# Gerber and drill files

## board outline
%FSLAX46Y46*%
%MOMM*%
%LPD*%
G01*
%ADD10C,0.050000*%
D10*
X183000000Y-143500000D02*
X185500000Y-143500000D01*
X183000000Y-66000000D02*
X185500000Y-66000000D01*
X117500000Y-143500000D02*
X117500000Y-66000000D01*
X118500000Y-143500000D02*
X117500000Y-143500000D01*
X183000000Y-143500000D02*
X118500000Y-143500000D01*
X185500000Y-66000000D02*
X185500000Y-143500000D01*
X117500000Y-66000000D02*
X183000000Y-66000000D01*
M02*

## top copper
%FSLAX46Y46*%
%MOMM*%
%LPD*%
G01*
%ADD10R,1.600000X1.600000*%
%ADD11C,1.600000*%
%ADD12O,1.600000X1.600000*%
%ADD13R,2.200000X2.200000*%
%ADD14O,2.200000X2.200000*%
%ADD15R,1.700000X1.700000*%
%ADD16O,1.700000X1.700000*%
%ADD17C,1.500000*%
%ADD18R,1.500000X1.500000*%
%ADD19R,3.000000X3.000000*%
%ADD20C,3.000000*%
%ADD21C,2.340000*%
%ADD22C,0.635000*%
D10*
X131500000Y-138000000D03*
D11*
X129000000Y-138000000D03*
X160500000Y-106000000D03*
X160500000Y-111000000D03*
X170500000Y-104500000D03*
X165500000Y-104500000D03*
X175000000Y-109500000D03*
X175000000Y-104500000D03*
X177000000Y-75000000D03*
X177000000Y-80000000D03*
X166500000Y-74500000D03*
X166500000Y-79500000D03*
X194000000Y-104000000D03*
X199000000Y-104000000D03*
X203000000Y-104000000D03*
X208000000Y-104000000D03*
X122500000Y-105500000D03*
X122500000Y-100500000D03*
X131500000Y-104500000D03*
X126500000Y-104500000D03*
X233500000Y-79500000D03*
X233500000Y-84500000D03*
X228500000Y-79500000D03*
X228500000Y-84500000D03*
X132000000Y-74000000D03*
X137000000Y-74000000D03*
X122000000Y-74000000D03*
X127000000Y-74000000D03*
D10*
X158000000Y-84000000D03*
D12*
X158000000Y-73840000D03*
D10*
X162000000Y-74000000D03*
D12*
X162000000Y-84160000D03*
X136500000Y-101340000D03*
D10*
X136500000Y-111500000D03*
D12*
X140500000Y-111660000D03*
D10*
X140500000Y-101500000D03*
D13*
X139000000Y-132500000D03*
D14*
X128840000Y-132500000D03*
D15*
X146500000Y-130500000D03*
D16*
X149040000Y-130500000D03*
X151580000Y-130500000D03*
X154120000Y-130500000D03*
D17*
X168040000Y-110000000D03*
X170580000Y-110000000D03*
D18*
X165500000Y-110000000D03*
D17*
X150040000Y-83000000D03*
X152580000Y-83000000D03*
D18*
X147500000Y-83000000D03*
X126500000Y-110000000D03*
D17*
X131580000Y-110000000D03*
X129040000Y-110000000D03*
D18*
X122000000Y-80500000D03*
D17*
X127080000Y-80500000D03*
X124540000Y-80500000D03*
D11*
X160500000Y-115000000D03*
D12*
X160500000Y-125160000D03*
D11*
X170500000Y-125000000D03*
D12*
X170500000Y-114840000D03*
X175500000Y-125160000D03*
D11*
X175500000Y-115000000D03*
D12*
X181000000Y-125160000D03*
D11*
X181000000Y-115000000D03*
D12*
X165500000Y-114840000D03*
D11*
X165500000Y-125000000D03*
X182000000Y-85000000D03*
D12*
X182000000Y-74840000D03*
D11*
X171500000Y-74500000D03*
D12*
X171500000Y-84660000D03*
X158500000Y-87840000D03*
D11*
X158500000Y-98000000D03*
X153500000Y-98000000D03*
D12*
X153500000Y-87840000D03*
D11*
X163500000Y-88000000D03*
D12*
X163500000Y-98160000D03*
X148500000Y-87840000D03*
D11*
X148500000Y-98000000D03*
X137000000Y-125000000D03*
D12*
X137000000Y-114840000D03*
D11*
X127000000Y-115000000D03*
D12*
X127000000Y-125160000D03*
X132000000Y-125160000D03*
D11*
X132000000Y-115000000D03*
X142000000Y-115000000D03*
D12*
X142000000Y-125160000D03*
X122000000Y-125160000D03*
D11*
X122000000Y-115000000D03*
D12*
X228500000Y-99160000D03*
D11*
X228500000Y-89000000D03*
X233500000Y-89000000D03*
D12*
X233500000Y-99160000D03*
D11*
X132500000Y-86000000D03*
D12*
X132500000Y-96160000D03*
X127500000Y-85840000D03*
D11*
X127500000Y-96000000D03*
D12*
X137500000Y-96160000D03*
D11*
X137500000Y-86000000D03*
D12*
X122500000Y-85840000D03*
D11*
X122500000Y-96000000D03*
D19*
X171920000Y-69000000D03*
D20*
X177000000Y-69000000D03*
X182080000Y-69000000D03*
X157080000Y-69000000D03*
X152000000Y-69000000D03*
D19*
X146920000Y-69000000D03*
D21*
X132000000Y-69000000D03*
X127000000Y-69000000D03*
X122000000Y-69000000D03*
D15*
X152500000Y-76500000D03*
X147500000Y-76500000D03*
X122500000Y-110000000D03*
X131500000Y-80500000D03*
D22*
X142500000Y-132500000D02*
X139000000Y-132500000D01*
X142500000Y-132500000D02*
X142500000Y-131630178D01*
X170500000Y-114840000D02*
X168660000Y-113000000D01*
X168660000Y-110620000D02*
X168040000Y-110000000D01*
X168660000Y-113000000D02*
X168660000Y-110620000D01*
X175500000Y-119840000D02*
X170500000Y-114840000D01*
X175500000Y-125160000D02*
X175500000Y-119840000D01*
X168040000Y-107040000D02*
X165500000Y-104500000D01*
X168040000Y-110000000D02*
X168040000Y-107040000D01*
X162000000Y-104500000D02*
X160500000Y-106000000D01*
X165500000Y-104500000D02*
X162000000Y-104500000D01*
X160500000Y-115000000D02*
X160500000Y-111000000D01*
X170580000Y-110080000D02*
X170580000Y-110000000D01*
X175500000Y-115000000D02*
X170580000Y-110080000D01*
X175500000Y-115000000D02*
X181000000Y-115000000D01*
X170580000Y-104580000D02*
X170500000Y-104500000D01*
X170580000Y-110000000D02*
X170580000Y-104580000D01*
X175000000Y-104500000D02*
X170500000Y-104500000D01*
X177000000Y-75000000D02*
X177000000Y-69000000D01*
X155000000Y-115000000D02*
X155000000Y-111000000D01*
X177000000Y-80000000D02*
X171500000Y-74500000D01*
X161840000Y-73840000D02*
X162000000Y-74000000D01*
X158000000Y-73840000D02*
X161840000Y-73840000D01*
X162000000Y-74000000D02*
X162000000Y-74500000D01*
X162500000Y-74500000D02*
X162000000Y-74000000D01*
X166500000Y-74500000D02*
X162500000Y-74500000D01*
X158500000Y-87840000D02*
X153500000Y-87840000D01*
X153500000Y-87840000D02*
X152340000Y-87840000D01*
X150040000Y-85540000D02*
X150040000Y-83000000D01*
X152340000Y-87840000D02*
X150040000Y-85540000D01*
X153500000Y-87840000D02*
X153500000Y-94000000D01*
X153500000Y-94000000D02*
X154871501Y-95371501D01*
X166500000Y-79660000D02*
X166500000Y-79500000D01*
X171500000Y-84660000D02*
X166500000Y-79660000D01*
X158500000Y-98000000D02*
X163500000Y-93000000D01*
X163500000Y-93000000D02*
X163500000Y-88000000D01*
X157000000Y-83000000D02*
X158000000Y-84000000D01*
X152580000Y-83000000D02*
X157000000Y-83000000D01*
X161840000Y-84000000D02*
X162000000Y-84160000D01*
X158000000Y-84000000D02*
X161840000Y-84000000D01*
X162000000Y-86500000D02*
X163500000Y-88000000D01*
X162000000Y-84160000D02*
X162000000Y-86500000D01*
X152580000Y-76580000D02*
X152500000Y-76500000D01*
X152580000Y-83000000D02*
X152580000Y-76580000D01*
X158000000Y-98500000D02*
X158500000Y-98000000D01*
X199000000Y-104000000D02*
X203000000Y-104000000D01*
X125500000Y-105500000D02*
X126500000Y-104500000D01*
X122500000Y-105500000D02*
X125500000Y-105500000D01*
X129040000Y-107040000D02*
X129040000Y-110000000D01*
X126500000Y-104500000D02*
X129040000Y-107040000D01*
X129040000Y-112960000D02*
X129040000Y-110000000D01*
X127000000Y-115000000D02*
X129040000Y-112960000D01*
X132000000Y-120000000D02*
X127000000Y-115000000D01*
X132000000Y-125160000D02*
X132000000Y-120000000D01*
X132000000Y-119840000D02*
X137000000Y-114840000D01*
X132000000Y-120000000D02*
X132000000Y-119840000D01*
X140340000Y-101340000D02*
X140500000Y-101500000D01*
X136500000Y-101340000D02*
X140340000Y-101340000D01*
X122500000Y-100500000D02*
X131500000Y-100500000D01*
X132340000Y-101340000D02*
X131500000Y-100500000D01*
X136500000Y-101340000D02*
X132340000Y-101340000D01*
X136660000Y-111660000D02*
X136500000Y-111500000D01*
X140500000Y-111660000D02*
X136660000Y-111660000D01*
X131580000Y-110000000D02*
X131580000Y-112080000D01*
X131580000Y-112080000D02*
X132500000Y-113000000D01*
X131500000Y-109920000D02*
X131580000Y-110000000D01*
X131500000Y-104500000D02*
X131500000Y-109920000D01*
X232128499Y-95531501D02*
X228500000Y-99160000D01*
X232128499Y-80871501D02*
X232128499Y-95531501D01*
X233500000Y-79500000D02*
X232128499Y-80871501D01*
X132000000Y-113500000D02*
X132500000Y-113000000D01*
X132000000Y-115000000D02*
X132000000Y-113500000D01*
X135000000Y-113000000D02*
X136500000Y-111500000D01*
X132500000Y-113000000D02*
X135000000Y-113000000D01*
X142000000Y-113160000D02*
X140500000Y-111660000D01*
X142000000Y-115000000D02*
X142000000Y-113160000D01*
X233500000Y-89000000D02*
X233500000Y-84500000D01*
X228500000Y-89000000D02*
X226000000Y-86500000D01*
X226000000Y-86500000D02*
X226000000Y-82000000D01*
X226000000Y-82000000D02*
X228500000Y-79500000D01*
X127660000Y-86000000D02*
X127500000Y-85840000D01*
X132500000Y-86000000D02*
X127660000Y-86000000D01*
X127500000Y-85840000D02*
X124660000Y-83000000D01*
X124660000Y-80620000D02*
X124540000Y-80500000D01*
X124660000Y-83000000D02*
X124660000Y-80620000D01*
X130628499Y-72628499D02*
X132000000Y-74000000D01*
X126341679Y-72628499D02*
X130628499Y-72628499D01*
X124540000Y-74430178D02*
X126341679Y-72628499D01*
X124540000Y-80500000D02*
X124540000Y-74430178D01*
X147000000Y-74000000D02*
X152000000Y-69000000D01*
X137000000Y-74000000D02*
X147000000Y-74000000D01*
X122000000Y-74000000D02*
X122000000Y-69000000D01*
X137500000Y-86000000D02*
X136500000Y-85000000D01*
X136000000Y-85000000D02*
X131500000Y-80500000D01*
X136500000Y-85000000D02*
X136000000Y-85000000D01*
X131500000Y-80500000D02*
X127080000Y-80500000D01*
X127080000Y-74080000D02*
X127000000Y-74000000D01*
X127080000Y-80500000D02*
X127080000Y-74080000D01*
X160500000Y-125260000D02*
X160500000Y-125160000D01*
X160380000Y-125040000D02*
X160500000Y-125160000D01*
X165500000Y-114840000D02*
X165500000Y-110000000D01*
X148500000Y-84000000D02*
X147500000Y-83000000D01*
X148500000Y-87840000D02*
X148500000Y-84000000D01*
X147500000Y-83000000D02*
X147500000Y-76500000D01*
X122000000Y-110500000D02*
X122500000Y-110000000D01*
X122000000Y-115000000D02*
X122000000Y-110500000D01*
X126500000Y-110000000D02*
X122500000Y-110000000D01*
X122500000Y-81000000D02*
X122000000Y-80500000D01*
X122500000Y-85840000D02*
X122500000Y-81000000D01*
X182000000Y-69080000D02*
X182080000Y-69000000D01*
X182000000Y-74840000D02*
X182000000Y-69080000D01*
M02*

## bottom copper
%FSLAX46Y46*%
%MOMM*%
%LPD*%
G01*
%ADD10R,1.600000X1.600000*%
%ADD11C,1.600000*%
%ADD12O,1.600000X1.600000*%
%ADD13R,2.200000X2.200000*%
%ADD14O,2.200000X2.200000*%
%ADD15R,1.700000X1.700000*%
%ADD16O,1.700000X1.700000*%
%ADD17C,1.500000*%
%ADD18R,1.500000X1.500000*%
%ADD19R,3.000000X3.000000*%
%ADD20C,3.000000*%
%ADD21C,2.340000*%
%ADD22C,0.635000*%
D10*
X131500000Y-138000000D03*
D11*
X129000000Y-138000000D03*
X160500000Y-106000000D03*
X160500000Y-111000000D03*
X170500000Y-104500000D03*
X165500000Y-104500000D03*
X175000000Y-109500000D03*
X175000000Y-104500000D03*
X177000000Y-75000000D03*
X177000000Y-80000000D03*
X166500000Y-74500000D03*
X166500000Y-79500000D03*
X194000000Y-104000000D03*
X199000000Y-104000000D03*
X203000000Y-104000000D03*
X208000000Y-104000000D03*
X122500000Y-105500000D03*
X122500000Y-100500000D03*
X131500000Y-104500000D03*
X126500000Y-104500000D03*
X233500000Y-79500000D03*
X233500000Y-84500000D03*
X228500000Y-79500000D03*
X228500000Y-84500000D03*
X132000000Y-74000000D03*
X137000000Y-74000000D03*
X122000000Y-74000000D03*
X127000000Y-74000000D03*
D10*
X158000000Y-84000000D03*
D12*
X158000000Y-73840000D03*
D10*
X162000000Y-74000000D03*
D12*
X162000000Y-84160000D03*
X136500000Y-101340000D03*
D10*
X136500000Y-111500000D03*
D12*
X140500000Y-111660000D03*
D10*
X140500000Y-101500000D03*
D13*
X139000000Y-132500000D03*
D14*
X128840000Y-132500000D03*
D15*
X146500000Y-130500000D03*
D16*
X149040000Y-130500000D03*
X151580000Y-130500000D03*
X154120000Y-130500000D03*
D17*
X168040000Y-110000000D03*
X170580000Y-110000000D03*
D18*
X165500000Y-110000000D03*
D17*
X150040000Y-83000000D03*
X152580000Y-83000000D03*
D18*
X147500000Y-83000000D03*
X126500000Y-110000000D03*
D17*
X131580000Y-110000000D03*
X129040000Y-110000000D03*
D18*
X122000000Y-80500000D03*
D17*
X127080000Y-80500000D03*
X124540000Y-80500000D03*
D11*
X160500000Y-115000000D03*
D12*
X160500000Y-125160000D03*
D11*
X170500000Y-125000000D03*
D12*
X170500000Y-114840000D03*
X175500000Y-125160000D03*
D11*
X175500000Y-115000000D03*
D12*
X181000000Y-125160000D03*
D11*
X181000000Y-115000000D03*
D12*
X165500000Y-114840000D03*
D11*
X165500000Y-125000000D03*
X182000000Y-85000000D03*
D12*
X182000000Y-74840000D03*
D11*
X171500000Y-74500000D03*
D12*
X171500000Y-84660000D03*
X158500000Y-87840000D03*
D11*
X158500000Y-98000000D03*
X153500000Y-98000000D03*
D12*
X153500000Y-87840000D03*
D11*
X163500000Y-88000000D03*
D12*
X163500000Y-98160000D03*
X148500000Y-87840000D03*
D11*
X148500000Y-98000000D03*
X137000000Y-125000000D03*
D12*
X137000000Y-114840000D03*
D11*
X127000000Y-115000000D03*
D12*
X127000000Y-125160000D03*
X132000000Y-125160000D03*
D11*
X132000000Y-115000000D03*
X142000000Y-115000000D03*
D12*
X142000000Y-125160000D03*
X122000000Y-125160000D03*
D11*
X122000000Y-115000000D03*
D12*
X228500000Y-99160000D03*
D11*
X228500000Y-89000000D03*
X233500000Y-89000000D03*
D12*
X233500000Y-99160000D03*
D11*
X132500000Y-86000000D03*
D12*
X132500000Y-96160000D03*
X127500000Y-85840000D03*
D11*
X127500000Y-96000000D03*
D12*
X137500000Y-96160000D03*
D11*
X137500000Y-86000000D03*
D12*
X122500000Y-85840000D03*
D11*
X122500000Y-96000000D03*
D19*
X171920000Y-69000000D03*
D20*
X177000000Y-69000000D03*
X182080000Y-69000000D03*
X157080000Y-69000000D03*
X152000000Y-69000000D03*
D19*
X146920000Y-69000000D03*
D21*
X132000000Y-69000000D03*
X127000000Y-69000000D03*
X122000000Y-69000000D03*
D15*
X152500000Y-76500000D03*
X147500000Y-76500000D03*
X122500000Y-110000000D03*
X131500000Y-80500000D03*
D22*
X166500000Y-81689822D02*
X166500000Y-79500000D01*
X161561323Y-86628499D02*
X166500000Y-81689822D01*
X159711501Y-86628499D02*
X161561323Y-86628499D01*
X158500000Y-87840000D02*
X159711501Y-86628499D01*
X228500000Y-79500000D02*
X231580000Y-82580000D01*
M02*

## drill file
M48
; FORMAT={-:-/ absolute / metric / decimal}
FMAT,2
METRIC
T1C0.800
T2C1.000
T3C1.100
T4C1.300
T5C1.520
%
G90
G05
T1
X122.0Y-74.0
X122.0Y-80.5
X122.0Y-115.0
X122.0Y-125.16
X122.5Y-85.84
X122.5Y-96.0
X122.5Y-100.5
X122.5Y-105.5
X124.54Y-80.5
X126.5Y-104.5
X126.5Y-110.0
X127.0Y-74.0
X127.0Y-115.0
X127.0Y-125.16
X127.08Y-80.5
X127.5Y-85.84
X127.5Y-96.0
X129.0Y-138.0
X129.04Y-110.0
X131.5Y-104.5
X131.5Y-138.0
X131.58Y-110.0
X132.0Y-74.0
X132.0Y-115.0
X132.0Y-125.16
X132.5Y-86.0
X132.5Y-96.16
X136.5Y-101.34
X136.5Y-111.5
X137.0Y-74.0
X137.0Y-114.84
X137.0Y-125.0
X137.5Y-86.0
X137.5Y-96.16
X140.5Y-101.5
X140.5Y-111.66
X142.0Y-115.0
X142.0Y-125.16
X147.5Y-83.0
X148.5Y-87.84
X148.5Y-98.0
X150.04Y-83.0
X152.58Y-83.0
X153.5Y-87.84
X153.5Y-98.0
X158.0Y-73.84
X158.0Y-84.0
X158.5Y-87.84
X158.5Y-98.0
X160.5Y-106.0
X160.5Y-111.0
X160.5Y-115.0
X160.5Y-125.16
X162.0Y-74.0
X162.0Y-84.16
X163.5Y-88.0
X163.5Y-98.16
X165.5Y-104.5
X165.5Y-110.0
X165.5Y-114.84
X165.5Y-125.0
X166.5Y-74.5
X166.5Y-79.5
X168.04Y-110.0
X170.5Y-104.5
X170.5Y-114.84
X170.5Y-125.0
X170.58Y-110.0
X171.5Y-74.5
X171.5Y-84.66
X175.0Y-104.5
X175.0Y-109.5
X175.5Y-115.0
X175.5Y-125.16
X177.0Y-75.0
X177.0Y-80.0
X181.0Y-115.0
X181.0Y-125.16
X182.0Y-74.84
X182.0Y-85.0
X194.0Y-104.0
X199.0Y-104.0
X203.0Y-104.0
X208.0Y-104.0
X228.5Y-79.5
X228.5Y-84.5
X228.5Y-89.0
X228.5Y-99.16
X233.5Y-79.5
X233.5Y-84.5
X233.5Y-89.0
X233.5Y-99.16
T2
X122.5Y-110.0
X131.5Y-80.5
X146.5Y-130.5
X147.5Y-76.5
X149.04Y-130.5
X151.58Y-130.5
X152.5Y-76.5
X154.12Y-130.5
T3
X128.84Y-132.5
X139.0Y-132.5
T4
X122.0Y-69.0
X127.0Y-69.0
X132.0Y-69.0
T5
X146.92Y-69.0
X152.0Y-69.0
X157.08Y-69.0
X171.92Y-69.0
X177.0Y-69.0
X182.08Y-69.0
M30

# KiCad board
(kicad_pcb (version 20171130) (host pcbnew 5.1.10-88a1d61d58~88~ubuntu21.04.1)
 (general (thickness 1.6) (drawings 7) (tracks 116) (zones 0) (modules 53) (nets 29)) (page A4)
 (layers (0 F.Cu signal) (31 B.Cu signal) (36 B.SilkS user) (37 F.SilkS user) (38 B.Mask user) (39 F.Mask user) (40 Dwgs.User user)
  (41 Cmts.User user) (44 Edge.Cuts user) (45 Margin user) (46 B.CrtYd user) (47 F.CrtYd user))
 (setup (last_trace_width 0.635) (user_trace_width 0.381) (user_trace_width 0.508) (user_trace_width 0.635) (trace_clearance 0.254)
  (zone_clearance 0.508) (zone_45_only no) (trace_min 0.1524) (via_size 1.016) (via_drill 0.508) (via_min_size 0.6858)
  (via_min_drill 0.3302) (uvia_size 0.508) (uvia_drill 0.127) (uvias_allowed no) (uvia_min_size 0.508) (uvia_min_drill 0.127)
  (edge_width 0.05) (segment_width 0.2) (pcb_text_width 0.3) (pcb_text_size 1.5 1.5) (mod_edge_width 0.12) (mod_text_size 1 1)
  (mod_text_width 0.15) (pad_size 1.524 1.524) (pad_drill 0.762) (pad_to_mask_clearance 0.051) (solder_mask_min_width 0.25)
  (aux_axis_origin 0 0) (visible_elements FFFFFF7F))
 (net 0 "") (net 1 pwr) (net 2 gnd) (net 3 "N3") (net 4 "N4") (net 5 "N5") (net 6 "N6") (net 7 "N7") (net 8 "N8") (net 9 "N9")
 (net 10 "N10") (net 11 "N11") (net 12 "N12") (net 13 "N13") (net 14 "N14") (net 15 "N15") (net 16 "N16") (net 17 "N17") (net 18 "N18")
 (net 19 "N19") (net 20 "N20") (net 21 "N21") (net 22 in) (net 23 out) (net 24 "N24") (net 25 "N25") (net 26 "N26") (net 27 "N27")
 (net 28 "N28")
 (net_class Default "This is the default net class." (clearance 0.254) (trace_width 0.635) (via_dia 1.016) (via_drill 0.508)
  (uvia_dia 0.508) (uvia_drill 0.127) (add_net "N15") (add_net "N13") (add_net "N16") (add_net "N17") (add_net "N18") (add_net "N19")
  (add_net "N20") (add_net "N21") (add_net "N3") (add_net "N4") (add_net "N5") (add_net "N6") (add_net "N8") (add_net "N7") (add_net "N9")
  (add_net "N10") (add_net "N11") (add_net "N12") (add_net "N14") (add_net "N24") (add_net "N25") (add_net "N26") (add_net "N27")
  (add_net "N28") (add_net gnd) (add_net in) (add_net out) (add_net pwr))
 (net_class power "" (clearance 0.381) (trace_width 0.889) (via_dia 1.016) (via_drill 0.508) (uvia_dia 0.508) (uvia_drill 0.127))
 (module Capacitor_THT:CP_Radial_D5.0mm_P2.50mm (layer F.Cu) (at 131.5 138 180)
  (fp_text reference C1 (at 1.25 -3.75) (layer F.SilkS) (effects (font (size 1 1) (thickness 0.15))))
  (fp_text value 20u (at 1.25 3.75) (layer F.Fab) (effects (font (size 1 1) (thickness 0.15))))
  (pad 1 thru_hole rect (at 0 0 180) (size 1.6 1.6) (drill 0.8) (layers *.Cu *.Mask) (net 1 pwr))
  (pad 2 thru_hole circle (at 2.5 0 180) (size 1.6 1.6) (drill 0.8) (layers *.Cu *.Mask) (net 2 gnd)))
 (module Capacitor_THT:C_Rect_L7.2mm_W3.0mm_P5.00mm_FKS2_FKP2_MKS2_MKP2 (layer F.Cu) (at 160.5 106 270)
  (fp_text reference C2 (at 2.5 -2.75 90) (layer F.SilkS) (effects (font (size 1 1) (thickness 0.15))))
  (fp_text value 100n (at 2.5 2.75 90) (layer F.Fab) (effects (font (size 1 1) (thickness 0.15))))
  (pad 1 thru_hole circle (at 0 0 270) (size 1.6 1.6) (drill 0.8) (layers *.Cu *.Mask) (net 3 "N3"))
  (pad 2 thru_hole circle (at 5 0 270) (size 1.6 1.6) (drill 0.8) (layers *.Cu *.Mask) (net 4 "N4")))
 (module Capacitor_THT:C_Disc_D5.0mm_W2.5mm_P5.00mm (layer F.Cu) (at 170.5 104.5 180)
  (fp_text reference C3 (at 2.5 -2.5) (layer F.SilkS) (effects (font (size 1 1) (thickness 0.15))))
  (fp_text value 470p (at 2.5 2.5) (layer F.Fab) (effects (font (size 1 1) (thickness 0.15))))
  (pad 1 thru_hole circle (at 0 0 180) (size 1.6 1.6) (drill 0.8) (layers *.Cu *.Mask) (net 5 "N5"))
  (pad 2 thru_hole circle (at 5 0 180) (size 1.6 1.6) (drill 0.8) (layers *.Cu *.Mask) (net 3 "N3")))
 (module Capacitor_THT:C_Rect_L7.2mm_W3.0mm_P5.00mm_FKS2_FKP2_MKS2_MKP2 (layer F.Cu) (at 175 109.5 90)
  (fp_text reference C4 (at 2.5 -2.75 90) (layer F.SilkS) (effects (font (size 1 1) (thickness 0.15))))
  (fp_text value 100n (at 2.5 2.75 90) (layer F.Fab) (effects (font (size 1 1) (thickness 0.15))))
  (pad 1 thru_hole circle (at 0 0 90) (size 1.6 1.6) (drill 0.8) (layers *.Cu *.Mask) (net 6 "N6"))
  (pad 2 thru_hole circle (at 5 0 90) (size 1.6 1.6) (drill 0.8) (layers *.Cu *.Mask) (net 5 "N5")))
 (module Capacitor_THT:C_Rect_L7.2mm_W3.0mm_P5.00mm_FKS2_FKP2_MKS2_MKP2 (layer F.Cu) (at 177 80 90)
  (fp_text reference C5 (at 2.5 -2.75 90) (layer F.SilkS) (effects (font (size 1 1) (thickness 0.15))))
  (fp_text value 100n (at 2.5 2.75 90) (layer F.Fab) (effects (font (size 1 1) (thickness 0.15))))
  (pad 2 thru_hole circle (at 5 0 90) (size 1.6 1.6) (drill 0.8) (layers *.Cu *.Mask) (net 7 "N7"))
  (pad 1 thru_hole circle (at 0 0 90) (size 1.6 1.6) (drill 0.8) (layers *.Cu *.Mask) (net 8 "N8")))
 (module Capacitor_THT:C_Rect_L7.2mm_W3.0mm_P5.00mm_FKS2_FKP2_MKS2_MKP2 (layer F.Cu) (at 166.5 74.5 270)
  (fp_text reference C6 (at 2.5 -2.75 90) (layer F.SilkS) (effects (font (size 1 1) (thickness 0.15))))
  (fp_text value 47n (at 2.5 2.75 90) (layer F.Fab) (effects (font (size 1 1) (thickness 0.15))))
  (pad 1 thru_hole circle (at 0 0 270) (size 1.6 1.6) (drill 0.8) (layers *.Cu *.Mask) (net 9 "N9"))
  (pad 2 thru_hole circle (at 5 0 270) (size 1.6 1.6) (drill 0.8) (layers *.Cu *.Mask) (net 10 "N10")))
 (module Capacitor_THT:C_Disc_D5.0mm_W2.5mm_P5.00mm (layer F.Cu) (at 199 104 180)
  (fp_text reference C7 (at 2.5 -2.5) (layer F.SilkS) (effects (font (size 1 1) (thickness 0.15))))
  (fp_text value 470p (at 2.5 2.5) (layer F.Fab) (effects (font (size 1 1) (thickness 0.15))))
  (pad 2 thru_hole circle (at 5 0 180) (size 1.6 1.6) (drill 0.8) (layers *.Cu *.Mask) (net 10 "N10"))
  (pad 1 thru_hole circle (at 0 0 180) (size 1.6 1.6) (drill 0.8) (layers *.Cu *.Mask) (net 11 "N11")))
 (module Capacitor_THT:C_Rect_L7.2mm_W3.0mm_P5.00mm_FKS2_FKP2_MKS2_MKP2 (layer F.Cu) (at 208 104 180)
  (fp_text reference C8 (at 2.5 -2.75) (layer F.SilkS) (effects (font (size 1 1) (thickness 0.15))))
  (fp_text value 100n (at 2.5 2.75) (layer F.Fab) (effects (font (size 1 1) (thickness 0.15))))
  (pad 2 thru_hole circle (at 5 0 180) (size 1.6 1.6) (drill 0.8) (layers *.Cu *.Mask) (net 11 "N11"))
  (pad 1 thru_hole circle (at 0 0 180) (size 1.6 1.6) (drill 0.8) (layers *.Cu *.Mask) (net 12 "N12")))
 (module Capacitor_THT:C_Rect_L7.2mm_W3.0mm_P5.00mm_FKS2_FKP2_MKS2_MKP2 (layer F.Cu) (at 122.5 100.5 270)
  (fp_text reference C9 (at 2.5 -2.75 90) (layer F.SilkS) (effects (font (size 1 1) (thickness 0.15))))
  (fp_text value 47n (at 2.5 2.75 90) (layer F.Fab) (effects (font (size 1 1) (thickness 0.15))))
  (pad 2 thru_hole circle (at 5 0 270) (size 1.6 1.6) (drill 0.8) (layers *.Cu *.Mask) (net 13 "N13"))
  (pad 1 thru_hole circle (at 0 0 270) (size 1.6 1.6) (drill 0.8) (layers *.Cu *.Mask) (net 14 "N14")))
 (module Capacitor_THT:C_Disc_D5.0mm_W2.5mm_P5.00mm (layer F.Cu) (at 131.5 104.5 180)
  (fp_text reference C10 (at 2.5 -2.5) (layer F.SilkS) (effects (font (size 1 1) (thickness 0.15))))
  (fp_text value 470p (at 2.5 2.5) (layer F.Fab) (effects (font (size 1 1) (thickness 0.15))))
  (pad 1 thru_hole circle (at 0 0 180) (size 1.6 1.6) (drill 0.8) (layers *.Cu *.Mask) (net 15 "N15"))
  (pad 2 thru_hole circle (at 5 0 180) (size 1.6 1.6) (drill 0.8) (layers *.Cu *.Mask) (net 13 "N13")))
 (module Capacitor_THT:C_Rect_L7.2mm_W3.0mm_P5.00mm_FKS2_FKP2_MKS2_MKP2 (layer F.Cu) (at 233.5 84.5 90)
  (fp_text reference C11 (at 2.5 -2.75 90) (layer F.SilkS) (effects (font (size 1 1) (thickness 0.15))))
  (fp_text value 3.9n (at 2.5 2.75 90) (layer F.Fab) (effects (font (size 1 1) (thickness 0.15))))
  (pad 2 thru_hole circle (at 5 0 90) (size 1.6 1.6) (drill 0.8) (layers *.Cu *.Mask) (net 15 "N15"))
  (pad 1 thru_hole circle (at 0 0 90) (size 1.6 1.6) (drill 0.8) (layers *.Cu *.Mask) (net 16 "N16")))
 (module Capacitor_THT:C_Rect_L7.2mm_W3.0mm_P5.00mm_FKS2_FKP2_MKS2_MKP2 (layer F.Cu) (at 228.5 84.5 90)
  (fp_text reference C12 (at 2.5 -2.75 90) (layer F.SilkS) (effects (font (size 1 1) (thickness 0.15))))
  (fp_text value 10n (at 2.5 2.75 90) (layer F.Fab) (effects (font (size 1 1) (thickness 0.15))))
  (pad 2 thru_hole circle (at 5 0 90) (size 1.6 1.6) (drill 0.8) (layers *.Cu *.Mask) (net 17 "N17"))
  (pad 1 thru_hole circle (at 0 0 90) (size 1.6 1.6) (drill 0.8) (layers *.Cu *.Mask) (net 2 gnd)))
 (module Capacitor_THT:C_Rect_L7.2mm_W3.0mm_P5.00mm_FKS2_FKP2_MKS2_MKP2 (layer F.Cu) (at 132 74)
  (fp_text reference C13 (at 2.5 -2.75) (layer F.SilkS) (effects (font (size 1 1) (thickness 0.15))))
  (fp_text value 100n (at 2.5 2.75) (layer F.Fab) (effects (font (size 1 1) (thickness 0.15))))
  (pad 1 thru_hole circle (at 0 0) (size 1.6 1.6) (drill 0.8) (layers *.Cu *.Mask) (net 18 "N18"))
  (pad 2 thru_hole circle (at 5 0) (size 1.6 1.6) (drill 0.8) (layers *.Cu *.Mask) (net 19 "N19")))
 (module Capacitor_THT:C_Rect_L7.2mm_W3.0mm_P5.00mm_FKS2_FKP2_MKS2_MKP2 (layer F.Cu) (at 122 74)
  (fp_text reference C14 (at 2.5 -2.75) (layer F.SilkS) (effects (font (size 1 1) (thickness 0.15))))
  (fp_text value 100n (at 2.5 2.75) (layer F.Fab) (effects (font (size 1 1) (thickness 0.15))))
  (pad 1 thru_hole circle (at 0 0) (size 1.6 1.6) (drill 0.8) (layers *.Cu *.Mask) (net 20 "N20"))
  (pad 2 thru_hole circle (at 5 0) (size 1.6 1.6) (drill 0.8) (layers *.Cu *.Mask) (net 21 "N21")))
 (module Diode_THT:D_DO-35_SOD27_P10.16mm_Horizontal (layer F.Cu) (at 158 84 90)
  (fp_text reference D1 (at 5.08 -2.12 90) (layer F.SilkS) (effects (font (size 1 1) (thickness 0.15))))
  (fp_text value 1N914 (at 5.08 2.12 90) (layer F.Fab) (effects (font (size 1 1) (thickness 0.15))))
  (pad 1 thru_hole rect (at 0 0 90) (size 1.6 1.6) (drill 0.8) (layers *.Cu *.Mask) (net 11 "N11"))
  (pad 2 thru_hole oval (at 10.16 0 90) (size 1.6 1.6) (drill 0.8) (layers *.Cu *.Mask) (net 9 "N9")))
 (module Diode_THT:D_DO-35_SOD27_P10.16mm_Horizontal (layer F.Cu) (at 162 74 270)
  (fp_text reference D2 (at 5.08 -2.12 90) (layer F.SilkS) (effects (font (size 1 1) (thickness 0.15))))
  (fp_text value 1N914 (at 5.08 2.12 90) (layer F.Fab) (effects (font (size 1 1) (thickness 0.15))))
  (pad 1 thru_hole rect (at 0 0 270) (size 1.6 1.6) (drill 0.8) (layers *.Cu *.Mask) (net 9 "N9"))
  (pad 2 thru_hole oval (at 10.16 0 270) (size 1.6 1.6) (drill 0.8) (layers *.Cu *.Mask) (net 11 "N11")))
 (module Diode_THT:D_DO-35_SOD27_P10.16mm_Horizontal (layer F.Cu) (at 136.5 111.5 90)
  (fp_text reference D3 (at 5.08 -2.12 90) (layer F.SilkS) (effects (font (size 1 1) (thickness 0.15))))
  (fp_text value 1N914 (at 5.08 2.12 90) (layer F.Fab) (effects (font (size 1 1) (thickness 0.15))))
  (pad 2 thru_hole oval (at 10.16 0 90) (size 1.6 1.6) (drill 0.8) (layers *.Cu *.Mask) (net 14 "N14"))
  (pad 1 thru_hole rect (at 0 0 90) (size 1.6 1.6) (drill 0.8) (layers *.Cu *.Mask) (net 15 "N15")))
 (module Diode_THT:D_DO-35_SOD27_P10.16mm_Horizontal (layer F.Cu) (at 140.5 101.5 270)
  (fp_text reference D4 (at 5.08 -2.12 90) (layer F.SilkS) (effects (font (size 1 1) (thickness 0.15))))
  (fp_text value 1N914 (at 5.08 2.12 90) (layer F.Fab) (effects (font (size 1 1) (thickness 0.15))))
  (pad 2 thru_hole oval (at 10.16 0 270) (size 1.6 1.6) (drill 0.8) (layers *.Cu *.Mask) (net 15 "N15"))
  (pad 1 thru_hole rect (at 0 0 270) (size 1.6 1.6) (drill 0.8) (layers *.Cu *.Mask) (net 14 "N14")))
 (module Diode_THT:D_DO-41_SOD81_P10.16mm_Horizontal (layer F.Cu) (at 139 132.5 180)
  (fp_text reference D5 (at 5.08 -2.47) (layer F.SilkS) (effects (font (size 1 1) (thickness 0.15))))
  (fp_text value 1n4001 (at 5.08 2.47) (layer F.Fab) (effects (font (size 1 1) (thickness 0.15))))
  (pad 1 thru_hole rect (at 0 0 180) (size 2.2 2.2) (drill 1.1) (layers *.Cu *.Mask) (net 1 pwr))
  (pad 2 thru_hole oval (at 10.16 0 180) (size 2.2 2.2) (drill 1.1) (layers *.Cu *.Mask) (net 2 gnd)))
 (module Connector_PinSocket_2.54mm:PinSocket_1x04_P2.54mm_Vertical (layer F.Cu) (at 146.5 130.5 90)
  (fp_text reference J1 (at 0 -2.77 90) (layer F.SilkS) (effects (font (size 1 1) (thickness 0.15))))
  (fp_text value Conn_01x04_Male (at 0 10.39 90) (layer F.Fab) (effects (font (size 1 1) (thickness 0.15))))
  (pad 1 thru_hole rect (at 0 0 90) (size 1.7 1.7) (drill 1) (layers *.Cu *.Mask) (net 1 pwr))
  (pad 2 thru_hole oval (at 0 2.54 90) (size 1.7 1.7) (drill 1) (layers *.Cu *.Mask) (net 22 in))
  (pad 3 thru_hole oval (at 0 5.08 90) (size 1.7 1.7) (drill 1) (layers *.Cu *.Mask) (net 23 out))
  (pad 4 thru_hole oval (at 0 7.62 90) (size 1.7 1.7) (drill 1) (layers *.Cu *.Mask) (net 2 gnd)))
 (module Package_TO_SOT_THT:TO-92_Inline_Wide (layer F.Cu) (at 165.5 110)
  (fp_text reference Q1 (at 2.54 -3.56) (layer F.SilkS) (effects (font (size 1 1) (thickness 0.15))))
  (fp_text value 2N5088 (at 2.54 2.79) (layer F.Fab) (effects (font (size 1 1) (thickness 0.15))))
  (pad 2 thru_hole circle (at 2.54 0) (size 1.5 1.5) (drill 0.8) (layers *.Cu *.Mask) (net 3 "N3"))
  (pad 3 thru_hole circle (at 5.08 0) (size 1.5 1.5) (drill 0.8) (layers *.Cu *.Mask) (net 5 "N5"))
  (pad 1 thru_hole rect (at 0 0) (size 1.5 1.5) (drill 0.8) (layers *.Cu *.Mask) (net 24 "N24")))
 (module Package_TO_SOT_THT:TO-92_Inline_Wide (layer F.Cu) (at 147.5 83)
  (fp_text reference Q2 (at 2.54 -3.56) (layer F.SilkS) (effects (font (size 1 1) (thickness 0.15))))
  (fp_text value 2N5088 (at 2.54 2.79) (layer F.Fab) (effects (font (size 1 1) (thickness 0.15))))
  (pad 2 thru_hole circle (at 2.54 0) (size 1.5 1.5) (drill 0.8) (layers *.Cu *.Mask) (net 10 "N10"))
  (pad 3 thru_hole circle (at 5.08 0) (size 1.5 1.5) (drill 0.8) (layers *.Cu *.Mask) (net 11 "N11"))
  (pad 1 thru_hole rect (at 0 0) (size 1.5 1.5) (drill 0.8) (layers *.Cu *.Mask) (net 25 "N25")))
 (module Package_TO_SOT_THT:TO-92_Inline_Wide (layer F.Cu) (at 126.5 110)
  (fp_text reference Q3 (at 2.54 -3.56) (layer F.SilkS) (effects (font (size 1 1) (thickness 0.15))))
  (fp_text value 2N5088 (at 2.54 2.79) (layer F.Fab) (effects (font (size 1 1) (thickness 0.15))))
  (pad 1 thru_hole rect (at 0 0) (size 1.5 1.5) (drill 0.8) (layers *.Cu *.Mask) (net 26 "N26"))
  (pad 3 thru_hole circle (at 5.08 0) (size 1.5 1.5) (drill 0.8) (layers *.Cu *.Mask) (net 15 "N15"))
  (pad 2 thru_hole circle (at 2.54 0) (size 1.5 1.5) (drill 0.8) (layers *.Cu *.Mask) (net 13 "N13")))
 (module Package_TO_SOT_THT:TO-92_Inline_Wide (layer F.Cu) (at 122 80.5)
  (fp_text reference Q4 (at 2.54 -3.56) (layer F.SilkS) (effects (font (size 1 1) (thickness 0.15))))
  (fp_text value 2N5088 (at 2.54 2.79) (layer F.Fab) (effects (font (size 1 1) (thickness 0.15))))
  (pad 1 thru_hole rect (at 0 0) (size 1.5 1.5) (drill 0.8) (layers *.Cu *.Mask) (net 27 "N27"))
  (pad 3 thru_hole circle (at 5.08 0) (size 1.5 1.5) (drill 0.8) (layers *.Cu *.Mask) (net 21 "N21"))
  (pad 2 thru_hole circle (at 2.54 0) (size 1.5 1.5) (drill 0.8) (layers *.Cu *.Mask) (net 18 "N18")))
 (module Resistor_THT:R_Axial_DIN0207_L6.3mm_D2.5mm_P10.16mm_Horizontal (layer F.Cu) (at 160.5 115 270)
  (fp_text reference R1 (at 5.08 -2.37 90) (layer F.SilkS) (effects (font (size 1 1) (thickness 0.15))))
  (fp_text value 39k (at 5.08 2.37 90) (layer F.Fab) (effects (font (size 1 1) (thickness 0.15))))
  (pad 1 thru_hole circle (at 0 0 270) (size 1.6 1.6) (drill 0.8) (layers *.Cu *.Mask) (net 4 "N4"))
  (pad 2 thru_hole oval (at 10.16 0 270) (size 1.6 1.6) (drill 0.8) (layers *.Cu *.Mask) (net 22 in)))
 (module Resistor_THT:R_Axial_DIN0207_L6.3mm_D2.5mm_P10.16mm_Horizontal (layer F.Cu) (at 170.5 125 90)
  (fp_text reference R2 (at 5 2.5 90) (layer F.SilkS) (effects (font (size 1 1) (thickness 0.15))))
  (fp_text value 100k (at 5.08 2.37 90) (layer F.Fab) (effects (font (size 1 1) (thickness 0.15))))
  (pad 1 thru_hole circle (at 0 0 90) (size 1.6 1.6) (drill 0.8) (layers *.Cu *.Mask) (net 2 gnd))
  (pad 2 thru_hole oval (at 10.16 0 90) (size 1.6 1.6) (drill 0.8) (layers *.Cu *.Mask) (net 3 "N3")))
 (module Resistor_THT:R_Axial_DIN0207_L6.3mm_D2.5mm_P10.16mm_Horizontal (layer F.Cu) (at 175.5 115 270)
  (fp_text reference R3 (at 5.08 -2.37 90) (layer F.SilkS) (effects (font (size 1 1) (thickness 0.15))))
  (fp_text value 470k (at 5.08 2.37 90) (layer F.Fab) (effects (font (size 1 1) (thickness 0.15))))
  (pad 2 thru_hole oval (at 10.16 0 270) (size 1.6 1.6) (drill 0.8) (layers *.Cu *.Mask) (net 3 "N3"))
  (pad 1 thru_hole circle (at 0 0 270) (size 1.6 1.6) (drill 0.8) (layers *.Cu *.Mask) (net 5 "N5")))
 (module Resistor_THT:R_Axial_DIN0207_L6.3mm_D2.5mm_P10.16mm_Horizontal (layer F.Cu) (at 181 115 270)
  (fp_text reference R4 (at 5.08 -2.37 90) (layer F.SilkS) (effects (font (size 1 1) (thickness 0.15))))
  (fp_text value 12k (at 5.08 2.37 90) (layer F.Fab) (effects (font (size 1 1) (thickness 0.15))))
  (pad 2 thru_hole oval (at 10.16 0 270) (size 1.6 1.6) (drill 0.8) (layers *.Cu *.Mask) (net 1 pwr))
  (pad 1 thru_hole circle (at 0 0 270) (size 1.6 1.6) (drill 0.8) (layers *.Cu *.Mask) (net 5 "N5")))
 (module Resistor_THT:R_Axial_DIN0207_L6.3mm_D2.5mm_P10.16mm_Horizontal (layer F.Cu) (at 165.5 125 90)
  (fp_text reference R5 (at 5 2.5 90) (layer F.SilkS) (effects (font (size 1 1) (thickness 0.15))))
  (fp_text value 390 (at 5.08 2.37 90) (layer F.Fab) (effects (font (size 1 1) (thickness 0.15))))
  (pad 2 thru_hole oval (at 10.16 0 90) (size 1.6 1.6) (drill 0.8) (layers *.Cu *.Mask) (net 24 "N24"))
  (pad 1 thru_hole circle (at 0 0 90) (size 1.6 1.6) (drill 0.8) (layers *.Cu *.Mask) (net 2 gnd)))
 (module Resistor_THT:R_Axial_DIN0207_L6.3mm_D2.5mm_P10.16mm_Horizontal (layer F.Cu) (at 182 85 90)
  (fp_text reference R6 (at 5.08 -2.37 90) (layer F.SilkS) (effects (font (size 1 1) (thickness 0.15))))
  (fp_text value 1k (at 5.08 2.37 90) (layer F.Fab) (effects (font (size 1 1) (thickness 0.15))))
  (pad 1 thru_hole circle (at 0 0 90) (size 1.6 1.6) (drill 0.8) (layers *.Cu *.Mask) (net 2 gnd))
  (pad 2 thru_hole oval (at 10.16 0 90) (size 1.6 1.6) (drill 0.8) (layers *.Cu *.Mask) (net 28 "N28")))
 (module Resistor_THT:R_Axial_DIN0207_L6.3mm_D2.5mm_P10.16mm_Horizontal (layer F.Cu) (at 171.5 74.5 270)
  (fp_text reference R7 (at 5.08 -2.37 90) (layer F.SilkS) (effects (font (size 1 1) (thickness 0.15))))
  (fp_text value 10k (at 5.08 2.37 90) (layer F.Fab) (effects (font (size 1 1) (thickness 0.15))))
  (pad 1 thru_hole circle (at 0 0 270) (size 1.6 1.6) (drill 0.8) (layers *.Cu *.Mask) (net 8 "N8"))
  (pad 2 thru_hole oval (at 10.16 0 270) (size 1.6 1.6) (drill 0.8) (layers *.Cu *.Mask) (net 10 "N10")))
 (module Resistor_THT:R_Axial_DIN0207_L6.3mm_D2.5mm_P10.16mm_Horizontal (layer F.Cu) (at 158.5 98 90)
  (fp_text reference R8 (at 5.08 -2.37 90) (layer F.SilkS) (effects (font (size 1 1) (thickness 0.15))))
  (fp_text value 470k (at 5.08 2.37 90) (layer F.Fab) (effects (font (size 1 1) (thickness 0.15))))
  (pad 2 thru_hole oval (at 10.16 0 90) (size 1.6 1.6) (drill 0.8) (layers *.Cu *.Mask) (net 10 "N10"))
  (pad 1 thru_hole circle (at 0 0 90) (size 1.6 1.6) (drill 0.8) (layers *.Cu *.Mask) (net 11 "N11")))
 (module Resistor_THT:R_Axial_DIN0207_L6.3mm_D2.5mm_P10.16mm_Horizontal (layer F.Cu) (at 153.5 98 90)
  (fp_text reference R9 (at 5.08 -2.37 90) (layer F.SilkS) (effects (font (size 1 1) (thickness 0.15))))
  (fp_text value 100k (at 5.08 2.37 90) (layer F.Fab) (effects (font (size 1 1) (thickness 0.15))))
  (pad 1 thru_hole circle (at 0 0 90) (size 1.6 1.6) (drill 0.8) (layers *.Cu *.Mask) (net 2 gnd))
  (pad 2 thru_hole oval (at 10.16 0 90) (size 1.6 1.6) (drill 0.8) (layers *.Cu *.Mask) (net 10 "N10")))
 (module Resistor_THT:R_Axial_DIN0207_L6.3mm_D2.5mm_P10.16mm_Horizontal (layer F.Cu) (at 163.5 88 270)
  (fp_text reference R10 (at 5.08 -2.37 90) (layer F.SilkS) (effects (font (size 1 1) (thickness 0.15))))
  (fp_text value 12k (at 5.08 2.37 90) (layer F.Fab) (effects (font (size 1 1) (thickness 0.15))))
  (pad 1 thru_hole circle (at 0 0 270) (size 1.6 1.6) (drill 0.8) (layers *.Cu *.Mask) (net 11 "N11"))
  (pad 2 thru_hole oval (at 10.16 0 270) (size 1.6 1.6) (drill 0.8) (layers *.Cu *.Mask) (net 1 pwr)))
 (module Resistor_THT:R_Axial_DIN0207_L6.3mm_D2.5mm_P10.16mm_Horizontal (layer F.Cu) (at 148.5 98 90)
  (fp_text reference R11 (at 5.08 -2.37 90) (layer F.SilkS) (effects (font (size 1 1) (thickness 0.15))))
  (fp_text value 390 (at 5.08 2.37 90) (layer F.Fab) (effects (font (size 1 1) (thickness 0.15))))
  (pad 2 thru_hole oval (at 10.16 0 90) (size 1.6 1.6) (drill 0.8) (layers *.Cu *.Mask) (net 25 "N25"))
  (pad 1 thru_hole circle (at 0 0 90) (size 1.6 1.6) (drill 0.8) (layers *.Cu *.Mask) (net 2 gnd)))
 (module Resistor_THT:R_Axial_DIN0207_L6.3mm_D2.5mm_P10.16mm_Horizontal (layer F.Cu) (at 137 125 90)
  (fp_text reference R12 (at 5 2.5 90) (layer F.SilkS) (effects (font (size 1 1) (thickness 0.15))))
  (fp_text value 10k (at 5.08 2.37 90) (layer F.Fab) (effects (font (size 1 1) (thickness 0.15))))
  (pad 1 thru_hole circle (at 0 0 90) (size 1.6 1.6) (drill 0.8) (layers *.Cu *.Mask) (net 12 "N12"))
  (pad 2 thru_hole oval (at 10.16 0 90) (size 1.6 1.6) (drill 0.8) (layers *.Cu *.Mask) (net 13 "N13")))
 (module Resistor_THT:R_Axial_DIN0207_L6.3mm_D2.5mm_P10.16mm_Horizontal (layer F.Cu) (at 127 115 270)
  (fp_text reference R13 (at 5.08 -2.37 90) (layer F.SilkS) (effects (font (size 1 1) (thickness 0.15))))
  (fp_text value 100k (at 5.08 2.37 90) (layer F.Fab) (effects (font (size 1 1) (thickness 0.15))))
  (pad 1 thru_hole circle (at 0 0 270) (size 1.6 1.6) (drill 0.8) (layers *.Cu *.Mask) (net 13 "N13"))
  (pad 2 thru_hole oval (at 10.16 0 270) (size 1.6 1.6) (drill 0.8) (layers *.Cu *.Mask) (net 2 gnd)))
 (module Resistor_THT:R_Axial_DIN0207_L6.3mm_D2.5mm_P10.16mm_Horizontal (layer F.Cu) (at 132 115 270)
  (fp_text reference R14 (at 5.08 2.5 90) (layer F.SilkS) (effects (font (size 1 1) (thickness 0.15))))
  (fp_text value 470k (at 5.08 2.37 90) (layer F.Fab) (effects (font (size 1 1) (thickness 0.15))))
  (pad 2 thru_hole oval (at 10.16 0 270) (size 1.6 1.6) (drill 0.8) (layers *.Cu *.Mask) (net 13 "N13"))
  (pad 1 thru_hole circle (at 0 0 270) (size 1.6 1.6) (drill 0.8) (layers *.Cu *.Mask) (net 15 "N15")))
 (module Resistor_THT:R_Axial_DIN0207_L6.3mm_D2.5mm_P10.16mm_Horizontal (layer F.Cu) (at 142 115 270)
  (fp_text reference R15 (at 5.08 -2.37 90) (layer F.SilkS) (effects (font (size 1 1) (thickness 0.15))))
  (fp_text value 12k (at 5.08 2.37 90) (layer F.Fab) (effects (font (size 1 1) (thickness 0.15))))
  (pad 1 thru_hole circle (at 0 0 270) (size 1.6 1.6) (drill 0.8) (layers *.Cu *.Mask) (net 15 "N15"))
  (pad 2 thru_hole oval (at 10.16 0 270) (size 1.6 1.6) (drill 0.8) (layers *.Cu *.Mask) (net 1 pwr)))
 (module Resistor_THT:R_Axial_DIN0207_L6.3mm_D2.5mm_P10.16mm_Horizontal (layer F.Cu) (at 122 115 270)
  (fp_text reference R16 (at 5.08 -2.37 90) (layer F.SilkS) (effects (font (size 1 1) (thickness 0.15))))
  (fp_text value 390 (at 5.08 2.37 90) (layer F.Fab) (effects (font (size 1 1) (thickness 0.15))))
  (pad 2 thru_hole oval (at 10.16 0 270) (size 1.6 1.6) (drill 0.8) (layers *.Cu *.Mask) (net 2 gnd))
  (pad 1 thru_hole circle (at 0 0 270) (size 1.6 1.6) (drill 0.8) (layers *.Cu *.Mask) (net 26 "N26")))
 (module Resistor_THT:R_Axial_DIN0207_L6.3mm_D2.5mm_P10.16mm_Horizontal (layer F.Cu) (at 228.5 89 270)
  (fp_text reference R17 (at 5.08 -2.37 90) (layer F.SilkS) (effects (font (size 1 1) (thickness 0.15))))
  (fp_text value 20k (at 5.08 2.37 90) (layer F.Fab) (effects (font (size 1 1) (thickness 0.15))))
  (pad 2 thru_hole oval (at 10.16 0 270) (size 1.6 1.6) (drill 0.8) (layers *.Cu *.Mask) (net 15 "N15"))
  (pad 1 thru_hole circle (at 0 0 270) (size 1.6 1.6) (drill 0.8) (layers *.Cu *.Mask) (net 17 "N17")))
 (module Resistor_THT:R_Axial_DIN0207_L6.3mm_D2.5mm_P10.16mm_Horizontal (layer F.Cu) (at 233.5 89 270)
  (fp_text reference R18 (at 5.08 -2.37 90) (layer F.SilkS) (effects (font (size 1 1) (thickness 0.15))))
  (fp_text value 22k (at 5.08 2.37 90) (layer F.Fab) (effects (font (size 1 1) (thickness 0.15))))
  (pad 1 thru_hole circle (at 0 0 270) (size 1.6 1.6) (drill 0.8) (layers *.Cu *.Mask) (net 16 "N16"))
  (pad 2 thru_hole oval (at 10.16 0 270) (size 1.6 1.6) (drill 0.8) (layers *.Cu *.Mask) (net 2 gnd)))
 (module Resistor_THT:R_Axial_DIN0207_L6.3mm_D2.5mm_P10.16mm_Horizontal (layer F.Cu) (at 132.5 86 270)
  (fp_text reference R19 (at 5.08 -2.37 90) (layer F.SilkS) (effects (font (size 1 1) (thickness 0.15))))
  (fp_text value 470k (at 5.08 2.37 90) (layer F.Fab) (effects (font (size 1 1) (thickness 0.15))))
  (pad 1 thru_hole circle (at 0 0 270) (size 1.6 1.6) (drill 0.8) (layers *.Cu *.Mask) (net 18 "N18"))
  (pad 2 thru_hole oval (at 10.16 0 270) (size 1.6 1.6) (drill 0.8) (layers *.Cu *.Mask) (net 1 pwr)))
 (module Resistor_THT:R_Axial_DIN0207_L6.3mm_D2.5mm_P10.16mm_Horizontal (layer F.Cu) (at 127.5 96 90)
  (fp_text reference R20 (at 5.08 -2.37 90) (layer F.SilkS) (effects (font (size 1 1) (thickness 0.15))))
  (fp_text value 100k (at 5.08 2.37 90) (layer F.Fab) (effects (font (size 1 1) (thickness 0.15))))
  (pad 2 thru_hole oval (at 10.16 0 90) (size 1.6 1.6) (drill 0.8) (layers *.Cu *.Mask) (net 18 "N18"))
  (pad 1 thru_hole circle (at 0 0 90) (size 1.6 1.6) (drill 0.8) (layers *.Cu *.Mask) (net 2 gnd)))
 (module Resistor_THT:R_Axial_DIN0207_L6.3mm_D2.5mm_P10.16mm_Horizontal (layer F.Cu) (at 137.5 86 270)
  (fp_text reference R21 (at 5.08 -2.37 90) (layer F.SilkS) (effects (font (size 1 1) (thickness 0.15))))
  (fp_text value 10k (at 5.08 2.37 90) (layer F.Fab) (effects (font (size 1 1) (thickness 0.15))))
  (pad 2 thru_hole oval (at 10.16 0 270) (size 1.6 1.6) (drill 0.8) (layers *.Cu *.Mask) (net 1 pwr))
  (pad 1 thru_hole circle (at 0 0 270) (size 1.6 1.6) (drill 0.8) (layers *.Cu *.Mask) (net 21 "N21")))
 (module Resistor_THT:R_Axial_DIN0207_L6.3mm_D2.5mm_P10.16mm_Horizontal (layer F.Cu) (at 122.5 96 90)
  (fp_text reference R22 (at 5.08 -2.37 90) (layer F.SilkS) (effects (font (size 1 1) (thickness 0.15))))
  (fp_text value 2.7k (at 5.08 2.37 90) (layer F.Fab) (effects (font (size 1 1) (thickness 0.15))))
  (pad 2 thru_hole oval (at 10.16 0 90) (size 1.6 1.6) (drill 0.8) (layers *.Cu *.Mask) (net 27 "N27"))
  (pad 1 thru_hole circle (at 0 0 90) (size 1.6 1.6) (drill 0.8) (layers *.Cu *.Mask) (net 2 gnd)))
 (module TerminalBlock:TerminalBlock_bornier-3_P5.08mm (layer B.Cu) (at 171.92 69)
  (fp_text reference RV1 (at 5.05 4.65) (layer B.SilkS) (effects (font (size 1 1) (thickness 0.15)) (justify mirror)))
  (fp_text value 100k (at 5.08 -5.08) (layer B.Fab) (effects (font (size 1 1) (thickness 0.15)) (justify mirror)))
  (pad 1 thru_hole rect (at 0 0) (size 3 3) (drill 1.52) (layers *.Cu *.Mask) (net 6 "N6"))
  (pad 2 thru_hole circle (at 5.08 0) (size 3 3) (drill 1.52) (layers *.Cu *.Mask) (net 7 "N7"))
  (pad 3 thru_hole circle (at 10.16 0) (size 3 3) (drill 1.52) (layers *.Cu *.Mask) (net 28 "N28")))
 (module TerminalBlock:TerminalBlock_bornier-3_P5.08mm (layer B.Cu) (at 146.92 69)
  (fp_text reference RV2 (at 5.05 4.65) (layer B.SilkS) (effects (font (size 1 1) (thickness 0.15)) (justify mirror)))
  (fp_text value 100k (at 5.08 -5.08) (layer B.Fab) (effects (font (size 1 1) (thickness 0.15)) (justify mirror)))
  (pad 3 thru_hole circle (at 10.16 0) (size 3 3) (drill 1.52) (layers *.Cu *.Mask) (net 17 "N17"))
  (pad 2 thru_hole circle (at 5.08 0) (size 3 3) (drill 1.52) (layers *.Cu *.Mask) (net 19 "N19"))
  (pad 1 thru_hole rect (at 0 0) (size 3 3) (drill 1.52) (layers *.Cu *.Mask) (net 16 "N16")))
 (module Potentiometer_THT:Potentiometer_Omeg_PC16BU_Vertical (layer B.Cu) (at 122 69 90)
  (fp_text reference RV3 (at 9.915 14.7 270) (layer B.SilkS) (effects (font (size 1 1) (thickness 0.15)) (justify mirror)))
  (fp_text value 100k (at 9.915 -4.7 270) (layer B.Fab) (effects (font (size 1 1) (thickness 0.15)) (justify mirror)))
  (pad 3 thru_hole circle (at 0 10 90) (size 2.34 2.34) (drill 1.3) (layers *.Cu *.Mask) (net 2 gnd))
  (pad 2 thru_hole circle (at 0 5 90) (size 2.34 2.34) (drill 1.3) (layers *.Cu *.Mask) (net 23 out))
  (pad 1 thru_hole circle (at 0 0 90) (size 2.34 2.34) (drill 1.3) (layers *.Cu *.Mask) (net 20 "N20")))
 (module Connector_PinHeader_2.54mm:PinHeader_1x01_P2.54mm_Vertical (layer F.Cu) (at 152.5 76.5)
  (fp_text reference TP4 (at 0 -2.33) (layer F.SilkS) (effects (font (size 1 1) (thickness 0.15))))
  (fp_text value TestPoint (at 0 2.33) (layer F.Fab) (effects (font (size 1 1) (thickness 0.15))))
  (pad 1 thru_hole rect (at 0 0) (size 1.7 1.7) (drill 1) (layers *.Cu *.Mask) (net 11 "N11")))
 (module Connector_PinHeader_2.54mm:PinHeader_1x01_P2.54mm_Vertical (layer F.Cu) (at 147.5 76.5 90)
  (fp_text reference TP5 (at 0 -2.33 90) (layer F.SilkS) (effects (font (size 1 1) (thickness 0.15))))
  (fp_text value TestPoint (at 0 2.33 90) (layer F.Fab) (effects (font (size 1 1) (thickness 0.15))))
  (pad 1 thru_hole rect (at 0 0 90) (size 1.7 1.7) (drill 1) (layers *.Cu *.Mask) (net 25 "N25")))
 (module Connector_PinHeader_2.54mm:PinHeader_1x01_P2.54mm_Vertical (layer F.Cu) (at 122.5 110)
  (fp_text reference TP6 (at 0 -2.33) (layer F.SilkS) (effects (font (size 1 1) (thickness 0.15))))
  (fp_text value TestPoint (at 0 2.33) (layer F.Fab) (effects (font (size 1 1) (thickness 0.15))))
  (pad 1 thru_hole rect (at 0 0) (size 1.7 1.7) (drill 1) (layers *.Cu *.Mask) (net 26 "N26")))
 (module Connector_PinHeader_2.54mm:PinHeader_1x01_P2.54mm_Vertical (layer F.Cu) (at 131.5 80.5)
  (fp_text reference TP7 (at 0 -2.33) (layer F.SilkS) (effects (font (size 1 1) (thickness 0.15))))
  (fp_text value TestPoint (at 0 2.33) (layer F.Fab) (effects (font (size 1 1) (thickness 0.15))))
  (pad 1 thru_hole rect (at 0 0) (size 1.7 1.7) (drill 1) (layers *.Cu *.Mask) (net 21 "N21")))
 (gr_line (start 183 143.5) (end 185.5 143.5) (layer Edge.Cuts) (width 0.05))
 (gr_line (start 183 66) (end 185.5 66) (layer Edge.Cuts) (width 0.05))
 (gr_line (start 117.5 143.5) (end 117.5 66) (layer Edge.Cuts) (width 0.05))
 (gr_line (start 118.5 143.5) (end 117.5 143.5) (layer Edge.Cuts) (width 0.05))
 (gr_line (start 183 143.5) (end 118.5 143.5) (layer Edge.Cuts) (width 0.05))
 (gr_line (start 185.5 66) (end 185.5 143.5) (layer Edge.Cuts) (width 0.05))
 (gr_line (start 117.5 66) (end 183 66) (layer Edge.Cuts) (width 0.05))
 (segment (start 142.5 132.5) (end 139 132.5) (width 0.635) (layer F.Cu) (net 1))
 (segment (start 142.5 132.5) (end 142.5 131.630178) (width 0.635) (layer F.Cu) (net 1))
 (segment (start 170.5 114.84) (end 168.66 113) (width 0.635) (layer F.Cu) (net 3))
 (segment (start 168.66 110.62) (end 168.04 110) (width 0.635) (layer F.Cu) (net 3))
 (segment (start 168.66 113) (end 168.66 110.62) (width 0.635) (layer F.Cu) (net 3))
 (segment (start 175.5 119.84) (end 170.5 114.84) (width 0.635) (layer F.Cu) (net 3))
 (segment (start 175.5 125.16) (end 175.5 119.84) (width 0.635) (layer F.Cu) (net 3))
 (segment (start 168.04 107.04) (end 165.5 104.5) (width 0.635) (layer F.Cu) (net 3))
 (segment (start 168.04 110) (end 168.04 107.04) (width 0.635) (layer F.Cu) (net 3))
 (segment (start 162 104.5) (end 160.5 106) (width 0.635) (layer F.Cu) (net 3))
 (segment (start 165.5 104.5) (end 162 104.5) (width 0.635) (layer F.Cu) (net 3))
 (segment (start 160.5 115) (end 160.5 111) (width 0.635) (layer F.Cu) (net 4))
 (segment (start 170.58 110.08) (end 170.58 110) (width 0.635) (layer F.Cu) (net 5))
 (segment (start 175.5 115) (end 170.58 110.08) (width 0.635) (layer F.Cu) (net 5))
 (segment (start 175.5 115) (end 181 115) (width 0.635) (layer F.Cu) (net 5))
 (segment (start 170.58 104.58) (end 170.5 104.5) (width 0.635) (layer F.Cu) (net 5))
 (segment (start 170.58 110) (end 170.58 104.58) (width 0.635) (layer F.Cu) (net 5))
 (segment (start 175 104.5) (end 170.5 104.5) (width 0.635) (layer F.Cu) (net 5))
 (segment (start 177 75) (end 177 69) (width 0.635) (layer F.Cu) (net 7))
 (segment (start 155 115) (end 155 111) (width 0.635) (layer F.Cu) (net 8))
 (segment (start 177 80) (end 171.5 74.5) (width 0.635) (layer F.Cu) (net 8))
 (segment (start 161.84 73.84) (end 162 74) (width 0.635) (layer F.Cu) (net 9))
 (segment (start 158 73.84) (end 161.84 73.84) (width 0.635) (layer F.Cu) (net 9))
 (segment (start 162 74) (end 162 74.5) (width 0.635) (layer F.Cu) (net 9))
 (segment (start 162.5 74.5) (end 162 74) (width 0.635) (layer F.Cu) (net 9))
 (segment (start 166.5 74.5) (end 162.5 74.5) (width 0.635) (layer F.Cu) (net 9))
 (segment (start 158.5 87.84) (end 153.5 87.84) (width 0.635) (layer F.Cu) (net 10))
 (segment (start 153.5 87.84) (end 152.34 87.84) (width 0.635) (layer F.Cu) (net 10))
 (segment (start 150.04 85.54) (end 150.04 83) (width 0.635) (layer F.Cu) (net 10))
 (segment (start 152.34 87.84) (end 150.04 85.54) (width 0.635) (layer F.Cu) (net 10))
 (segment (start 153.5 87.84) (end 153.5 94) (width 0.635) (layer F.Cu) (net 10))
 (segment (start 153.5 94) (end 154.871501 95.371501) (width 0.635) (layer F.Cu) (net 10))
 (segment (start 166.5 81.689822) (end 166.5 79.5) (width 0.635) (layer B.Cu) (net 10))
 (segment (start 161.561323 86.628499) (end 166.5 81.689822) (width 0.635) (layer B.Cu) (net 10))
 (segment (start 159.711501 86.628499) (end 161.561323 86.628499) (width 0.635) (layer B.Cu) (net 10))
 (segment (start 158.5 87.84) (end 159.711501 86.628499) (width 0.635) (layer B.Cu) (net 10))
 (segment (start 166.5 79.66) (end 166.5 79.5) (width 0.635) (layer F.Cu) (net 10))
 (segment (start 171.5 84.66) (end 166.5 79.66) (width 0.635) (layer F.Cu) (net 10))
 (segment (start 158.5 98) (end 163.5 93) (width 0.635) (layer F.Cu) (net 11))
 (segment (start 163.5 93) (end 163.5 88) (width 0.635) (layer F.Cu) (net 11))
 (segment (start 157 83) (end 158 84) (width 0.635) (layer F.Cu) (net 11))
 (segment (start 152.58 83) (end 157 83) (width 0.635) (layer F.Cu) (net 11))
 (segment (start 161.84 84) (end 162 84.16) (width 0.635) (layer F.Cu) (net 11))
 (segment (start 158 84) (end 161.84 84) (width 0.635) (layer F.Cu) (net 11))
 (segment (start 162 86.5) (end 163.5 88) (width 0.635) (layer F.Cu) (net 11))
 (segment (start 162 84.16) (end 162 86.5) (width 0.635) (layer F.Cu) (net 11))
 (segment (start 152.58 76.58) (end 152.5 76.5) (width 0.635) (layer F.Cu) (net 11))
 (segment (start 152.58 83) (end 152.58 76.58) (width 0.635) (layer F.Cu) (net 11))
 (segment (start 158 98.5) (end 158.5 98) (width 0.635) (layer F.Cu) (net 11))
 (segment (start 199 104) (end 203 104) (width 0.635) (layer F.Cu) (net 11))
 (segment (start 125.5 105.5) (end 126.5 104.5) (width 0.635) (layer F.Cu) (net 13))
 (segment (start 122.5 105.5) (end 125.5 105.5) (width 0.635) (layer F.Cu) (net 13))
 (segment (start 129.04 107.04) (end 129.04 110) (width 0.635) (layer F.Cu) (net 13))
 (segment (start 126.5 104.5) (end 129.04 107.04) (width 0.635) (layer F.Cu) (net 13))
 (segment (start 129.04 112.96) (end 129.04 110) (width 0.635) (layer F.Cu) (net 13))
 (segment (start 127 115) (end 129.04 112.96) (width 0.635) (layer F.Cu) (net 13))
 (segment (start 132 120) (end 127 115) (width 0.635) (layer F.Cu) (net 13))
 (segment (start 132 125.16) (end 132 120) (width 0.635) (layer F.Cu) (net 13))
 (segment (start 132 119.84) (end 137 114.84) (width 0.635) (layer F.Cu) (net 13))
 (segment (start 132 120) (end 132 119.84) (width 0.635) (layer F.Cu) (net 13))
 (segment (start 140.34 101.34) (end 140.5 101.5) (width 0.635) (layer F.Cu) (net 14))
 (segment (start 136.5 101.34) (end 140.34 101.34) (width 0.635) (layer F.Cu) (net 14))
 (segment (start 122.5 100.5) (end 131.5 100.5) (width 0.635) (layer F.Cu) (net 14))
 (segment (start 132.34 101.34) (end 131.5 100.5) (width 0.635) (layer F.Cu) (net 14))
 (segment (start 136.5 101.34) (end 132.34 101.34) (width 0.635) (layer F.Cu) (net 14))
 (segment (start 136.66 111.66) (end 136.5 111.5) (width 0.635) (layer F.Cu) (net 15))
 (segment (start 140.5 111.66) (end 136.66 111.66) (width 0.635) (layer F.Cu) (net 15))
 (segment (start 131.58 110) (end 131.58 112.08) (width 0.635) (layer F.Cu) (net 15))
 (segment (start 131.58 112.08) (end 132.5 113) (width 0.635) (layer F.Cu) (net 15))
 (segment (start 131.5 109.92) (end 131.58 110) (width 0.635) (layer F.Cu) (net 15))
 (segment (start 131.5 104.5) (end 131.5 109.92) (width 0.635) (layer F.Cu) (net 15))
 (segment (start 232.128499 95.531501) (end 228.5 99.16) (width 0.635) (layer F.Cu) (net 15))
 (segment (start 232.128499 80.871501) (end 232.128499 95.531501) (width 0.635) (layer F.Cu) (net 15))
 (segment (start 233.5 79.5) (end 232.128499 80.871501) (width 0.635) (layer F.Cu) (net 15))
 (segment (start 132 113.5) (end 132.5 113) (width 0.635) (layer F.Cu) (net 15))
 (segment (start 132 115) (end 132 113.5) (width 0.635) (layer F.Cu) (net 15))
 (segment (start 135 113) (end 136.5 111.5) (width 0.635) (layer F.Cu) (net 15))
 (segment (start 132.5 113) (end 135 113) (width 0.635) (layer F.Cu) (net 15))
 (segment (start 142 113.16) (end 140.5 111.66) (width 0.635) (layer F.Cu) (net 15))
 (segment (start 142 115) (end 142 113.16) (width 0.635) (layer F.Cu) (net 15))
 (segment (start 233.5 89) (end 233.5 84.5) (width 0.635) (layer F.Cu) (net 16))
 (segment (start 228.5 89) (end 226 86.5) (width 0.635) (layer F.Cu) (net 17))
 (segment (start 226 86.5) (end 226 82) (width 0.635) (layer F.Cu) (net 17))
 (segment (start 226 82) (end 228.5 79.5) (width 0.635) (layer F.Cu) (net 17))
 (segment (start 228.5 79.5) (end 231.58 82.58) (width 0.635) (layer B.Cu) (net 17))
 (segment (start 127.66 86) (end 127.5 85.84) (width 0.635) (layer F.Cu) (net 18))
 (segment (start 132.5 86) (end 127.66 86) (width 0.635) (layer F.Cu) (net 18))
 (segment (start 127.5 85.84) (end 124.66 83) (width 0.635) (layer F.Cu) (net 18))
 (segment (start 124.66 80.62) (end 124.54 80.5) (width 0.635) (layer F.Cu) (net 18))
 (segment (start 124.66 83) (end 124.66 80.62) (width 0.635) (layer F.Cu) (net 18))
 (segment (start 130.628499 72.628499) (end 132 74) (width 0.635) (layer F.Cu) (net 18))
 (segment (start 126.341679 72.628499) (end 130.628499 72.628499) (width 0.635) (layer F.Cu) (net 18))
 (segment (start 124.54 74.430178) (end 126.341679 72.628499) (width 0.635) (layer F.Cu) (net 18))
 (segment (start 124.54 80.5) (end 124.54 74.430178) (width 0.635) (layer F.Cu) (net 18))
 (segment (start 147 74) (end 152 69) (width 0.635) (layer F.Cu) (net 19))
 (segment (start 137 74) (end 147 74) (width 0.635) (layer F.Cu) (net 19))
 (segment (start 122 74) (end 122 69) (width 0.635) (layer F.Cu) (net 20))
 (segment (start 137.5 86) (end 136.5 85) (width 0.635) (layer F.Cu) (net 21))
 (segment (start 136 85) (end 131.5 80.5) (width 0.635) (layer F.Cu) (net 21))
 (segment (start 136.5 85) (end 136 85) (width 0.635) (layer F.Cu) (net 21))
 (segment (start 131.5 80.5) (end 127.08 80.5) (width 0.635) (layer F.Cu) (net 21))
 (segment (start 127.08 74.08) (end 127 74) (width 0.635) (layer F.Cu) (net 21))
 (segment (start 127.08 80.5) (end 127.08 74.08) (width 0.635) (layer F.Cu) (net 21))
 (segment (start 160.5 125.26) (end 160.5 125.16) (width 0.635) (layer F.Cu) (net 22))
 (segment (start 160.38 125.04) (end 160.5 125.16) (width 0.635) (layer F.Cu) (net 22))
 (segment (start 165.5 114.84) (end 165.5 110) (width 0.635) (layer F.Cu) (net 24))
 (segment (start 148.5 84) (end 147.5 83) (width 0.635) (layer F.Cu) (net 25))
 (segment (start 148.5 87.84) (end 148.5 84) (width 0.635) (layer F.Cu) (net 25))
 (segment (start 147.5 83) (end 147.5 76.5) (width 0.635) (layer F.Cu) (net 25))
 (segment (start 122 110.5) (end 122.5 110) (width 0.635) (layer F.Cu) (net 26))
 (segment (start 122 115) (end 122 110.5) (width 0.635) (layer F.Cu) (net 26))
 (segment (start 126.5 110) (end 122.5 110) (width 0.635) (layer F.Cu) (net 26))
 (segment (start 122.5 81) (end 122 80.5) (width 0.635) (layer F.Cu) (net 27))
 (segment (start 122.5 85.84) (end 122.5 81) (width 0.635) (layer F.Cu) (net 27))
 (segment (start 182 69.08) (end 182.08 69) (width 0.635) (layer F.Cu) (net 28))
 (segment (start 182 74.84) (end 182 69.08) (width 0.635) (layer F.Cu) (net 28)))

